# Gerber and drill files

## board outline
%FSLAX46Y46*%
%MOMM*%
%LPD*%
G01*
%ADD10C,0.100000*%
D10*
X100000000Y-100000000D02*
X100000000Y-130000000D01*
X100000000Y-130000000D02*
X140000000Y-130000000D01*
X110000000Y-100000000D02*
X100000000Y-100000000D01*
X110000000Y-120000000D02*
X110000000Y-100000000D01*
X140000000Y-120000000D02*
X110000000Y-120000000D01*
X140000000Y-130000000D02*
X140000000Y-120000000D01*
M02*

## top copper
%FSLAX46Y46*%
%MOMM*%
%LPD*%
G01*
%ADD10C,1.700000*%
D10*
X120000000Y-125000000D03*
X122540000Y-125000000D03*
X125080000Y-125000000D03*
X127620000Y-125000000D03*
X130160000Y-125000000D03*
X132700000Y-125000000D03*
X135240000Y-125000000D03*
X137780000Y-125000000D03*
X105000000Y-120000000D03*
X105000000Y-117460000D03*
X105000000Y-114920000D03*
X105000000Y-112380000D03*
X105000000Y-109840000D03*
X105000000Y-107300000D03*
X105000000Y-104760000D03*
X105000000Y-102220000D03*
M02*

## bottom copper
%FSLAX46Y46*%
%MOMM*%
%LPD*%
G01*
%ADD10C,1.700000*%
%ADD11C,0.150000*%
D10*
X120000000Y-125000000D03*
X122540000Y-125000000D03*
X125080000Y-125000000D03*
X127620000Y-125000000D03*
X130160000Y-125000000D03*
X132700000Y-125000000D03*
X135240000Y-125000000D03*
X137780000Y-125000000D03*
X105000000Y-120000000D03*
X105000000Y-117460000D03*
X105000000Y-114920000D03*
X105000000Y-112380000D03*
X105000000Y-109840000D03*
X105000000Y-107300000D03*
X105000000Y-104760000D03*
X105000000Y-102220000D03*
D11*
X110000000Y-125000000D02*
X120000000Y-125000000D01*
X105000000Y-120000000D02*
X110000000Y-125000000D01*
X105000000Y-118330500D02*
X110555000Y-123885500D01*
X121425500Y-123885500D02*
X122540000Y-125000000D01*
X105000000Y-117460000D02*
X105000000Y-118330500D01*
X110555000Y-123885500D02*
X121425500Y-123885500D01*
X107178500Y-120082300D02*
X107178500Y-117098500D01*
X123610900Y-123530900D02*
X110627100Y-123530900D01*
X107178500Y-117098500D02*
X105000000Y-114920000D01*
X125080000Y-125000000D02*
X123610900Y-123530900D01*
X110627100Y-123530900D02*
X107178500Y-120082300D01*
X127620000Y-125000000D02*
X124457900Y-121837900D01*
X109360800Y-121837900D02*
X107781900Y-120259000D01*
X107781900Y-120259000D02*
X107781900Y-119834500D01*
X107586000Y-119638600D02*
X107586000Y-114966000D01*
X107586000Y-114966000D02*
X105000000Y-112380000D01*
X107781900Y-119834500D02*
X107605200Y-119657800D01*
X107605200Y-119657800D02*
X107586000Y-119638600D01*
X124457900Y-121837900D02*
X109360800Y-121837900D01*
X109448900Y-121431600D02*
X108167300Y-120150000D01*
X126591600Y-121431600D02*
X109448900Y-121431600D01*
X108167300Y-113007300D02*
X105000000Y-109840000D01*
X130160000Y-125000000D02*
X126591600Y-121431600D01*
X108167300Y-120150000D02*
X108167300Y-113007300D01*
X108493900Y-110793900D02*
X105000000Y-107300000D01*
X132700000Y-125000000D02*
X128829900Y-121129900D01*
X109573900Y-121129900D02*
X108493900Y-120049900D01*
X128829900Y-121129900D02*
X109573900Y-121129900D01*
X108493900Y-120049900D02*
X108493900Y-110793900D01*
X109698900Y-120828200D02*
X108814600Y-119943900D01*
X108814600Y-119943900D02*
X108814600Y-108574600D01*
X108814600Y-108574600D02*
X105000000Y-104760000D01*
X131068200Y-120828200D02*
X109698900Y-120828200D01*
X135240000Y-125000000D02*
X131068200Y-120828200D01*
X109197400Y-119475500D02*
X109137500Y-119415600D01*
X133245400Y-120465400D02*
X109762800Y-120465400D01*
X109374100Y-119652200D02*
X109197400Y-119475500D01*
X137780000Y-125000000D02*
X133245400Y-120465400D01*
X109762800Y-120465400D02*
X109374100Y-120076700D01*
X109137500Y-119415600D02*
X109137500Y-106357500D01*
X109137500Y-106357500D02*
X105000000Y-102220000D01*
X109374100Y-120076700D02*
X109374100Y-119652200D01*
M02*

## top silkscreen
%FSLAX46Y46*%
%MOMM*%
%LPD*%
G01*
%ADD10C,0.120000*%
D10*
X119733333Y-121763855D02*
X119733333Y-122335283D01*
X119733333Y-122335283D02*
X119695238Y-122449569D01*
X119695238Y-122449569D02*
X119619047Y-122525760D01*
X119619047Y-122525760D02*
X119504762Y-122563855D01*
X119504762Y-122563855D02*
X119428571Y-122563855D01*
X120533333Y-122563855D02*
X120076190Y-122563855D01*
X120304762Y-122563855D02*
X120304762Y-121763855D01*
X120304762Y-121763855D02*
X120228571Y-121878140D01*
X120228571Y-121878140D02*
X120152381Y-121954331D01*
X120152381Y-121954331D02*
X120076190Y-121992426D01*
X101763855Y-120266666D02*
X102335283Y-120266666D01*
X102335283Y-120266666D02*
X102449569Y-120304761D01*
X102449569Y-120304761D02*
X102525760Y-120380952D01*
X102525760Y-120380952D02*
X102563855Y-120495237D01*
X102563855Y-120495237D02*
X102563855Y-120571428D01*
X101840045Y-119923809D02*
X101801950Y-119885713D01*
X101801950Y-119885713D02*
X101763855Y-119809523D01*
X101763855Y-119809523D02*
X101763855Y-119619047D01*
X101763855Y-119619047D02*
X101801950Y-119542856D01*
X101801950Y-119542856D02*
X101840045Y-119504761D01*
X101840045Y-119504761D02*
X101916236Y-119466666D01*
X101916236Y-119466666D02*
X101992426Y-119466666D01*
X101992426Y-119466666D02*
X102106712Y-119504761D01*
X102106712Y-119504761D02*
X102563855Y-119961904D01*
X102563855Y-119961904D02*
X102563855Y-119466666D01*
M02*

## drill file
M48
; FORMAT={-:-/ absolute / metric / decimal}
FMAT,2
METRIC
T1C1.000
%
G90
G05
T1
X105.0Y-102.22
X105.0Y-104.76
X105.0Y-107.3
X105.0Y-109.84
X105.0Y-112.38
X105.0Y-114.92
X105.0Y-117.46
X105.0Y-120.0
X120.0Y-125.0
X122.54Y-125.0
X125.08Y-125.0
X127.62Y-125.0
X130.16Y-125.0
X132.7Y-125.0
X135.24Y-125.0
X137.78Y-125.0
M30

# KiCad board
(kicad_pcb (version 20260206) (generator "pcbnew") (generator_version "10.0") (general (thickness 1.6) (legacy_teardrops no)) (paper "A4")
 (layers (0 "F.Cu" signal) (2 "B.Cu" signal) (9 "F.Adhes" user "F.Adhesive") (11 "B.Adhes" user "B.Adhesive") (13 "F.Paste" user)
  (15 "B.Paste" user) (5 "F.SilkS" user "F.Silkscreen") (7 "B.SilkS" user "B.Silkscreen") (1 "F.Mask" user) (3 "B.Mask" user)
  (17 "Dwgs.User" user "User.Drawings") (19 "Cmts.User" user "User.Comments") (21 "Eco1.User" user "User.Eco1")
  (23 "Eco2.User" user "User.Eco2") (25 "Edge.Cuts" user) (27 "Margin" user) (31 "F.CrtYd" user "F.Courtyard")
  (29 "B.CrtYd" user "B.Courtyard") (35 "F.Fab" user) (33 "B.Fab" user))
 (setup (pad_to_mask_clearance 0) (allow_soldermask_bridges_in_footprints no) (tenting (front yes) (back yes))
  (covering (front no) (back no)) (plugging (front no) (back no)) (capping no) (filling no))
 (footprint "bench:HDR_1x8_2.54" (layer "F.Cu") (at 120 125)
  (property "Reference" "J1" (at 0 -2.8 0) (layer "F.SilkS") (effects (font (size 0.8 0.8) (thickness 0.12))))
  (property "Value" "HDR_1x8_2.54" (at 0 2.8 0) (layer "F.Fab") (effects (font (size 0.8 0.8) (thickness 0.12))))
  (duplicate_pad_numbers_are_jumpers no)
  (pad "1" thru_hole circle (at 0 0) (size 1.7 1.7) (drill 1) (layers "*.Cu" "*.Mask") (remove_unused_layers no) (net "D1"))
  (pad "2" thru_hole circle (at 2.54 0) (size 1.7 1.7) (drill 1) (layers "*.Cu" "*.Mask") (remove_unused_layers no) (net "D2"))
  (pad "3" thru_hole circle (at 5.08 0) (size 1.7 1.7) (drill 1) (layers "*.Cu" "*.Mask") (remove_unused_layers no) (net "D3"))
  (pad "4" thru_hole circle (at 7.62 0) (size 1.7 1.7) (drill 1) (layers "*.Cu" "*.Mask") (remove_unused_layers no) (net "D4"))
  (pad "5" thru_hole circle (at 10.16 0) (size 1.7 1.7) (drill 1) (layers "*.Cu" "*.Mask") (remove_unused_layers no) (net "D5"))
  (pad "6" thru_hole circle (at 12.7 0) (size 1.7 1.7) (drill 1) (layers "*.Cu" "*.Mask") (remove_unused_layers no) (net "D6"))
  (pad "7" thru_hole circle (at 15.24 0) (size 1.7 1.7) (drill 1) (layers "*.Cu" "*.Mask") (remove_unused_layers no) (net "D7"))
  (pad "8" thru_hole circle (at 17.78 0) (size 1.7 1.7) (drill 1) (layers "*.Cu" "*.Mask") (remove_unused_layers no) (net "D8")))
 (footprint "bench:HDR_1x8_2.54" (layer "F.Cu") (at 105 120 90)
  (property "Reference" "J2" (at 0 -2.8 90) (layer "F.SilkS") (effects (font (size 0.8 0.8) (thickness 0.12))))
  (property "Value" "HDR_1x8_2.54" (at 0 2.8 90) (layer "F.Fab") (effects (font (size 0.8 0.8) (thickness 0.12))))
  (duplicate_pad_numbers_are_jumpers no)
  (pad "1" thru_hole circle (at 0 0 90) (size 1.7 1.7) (drill 1) (layers "*.Cu" "*.Mask") (remove_unused_layers no) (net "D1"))
  (pad "2" thru_hole circle (at 2.54 0 90) (size 1.7 1.7) (drill 1) (layers "*.Cu" "*.Mask") (remove_unused_layers no) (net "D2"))
  (pad "3" thru_hole circle (at 5.08 0 90) (size 1.7 1.7) (drill 1) (layers "*.Cu" "*.Mask") (remove_unused_layers no) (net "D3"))
  (pad "4" thru_hole circle (at 7.62 0 90) (size 1.7 1.7) (drill 1) (layers "*.Cu" "*.Mask") (remove_unused_layers no) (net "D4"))
  (pad "5" thru_hole circle (at 10.16 0 90) (size 1.7 1.7) (drill 1) (layers "*.Cu" "*.Mask") (remove_unused_layers no) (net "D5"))
  (pad "6" thru_hole circle (at 12.7 0 90) (size 1.7 1.7) (drill 1) (layers "*.Cu" "*.Mask") (remove_unused_layers no) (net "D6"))
  (pad "7" thru_hole circle (at 15.24 0 90) (size 1.7 1.7) (drill 1) (layers "*.Cu" "*.Mask") (remove_unused_layers no) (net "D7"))
  (pad "8" thru_hole circle (at 17.78 0 90) (size 1.7 1.7) (drill 1) (layers "*.Cu" "*.Mask") (remove_unused_layers no) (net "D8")))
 (gr_line (start 100 100) (end 100 130) (stroke (width 0.1) (type solid)) (layer "Edge.Cuts"))
 (gr_line (start 100 130) (end 140 130) (stroke (width 0.1) (type solid)) (layer "Edge.Cuts"))
 (gr_line (start 110 100) (end 100 100) (stroke (width 0.1) (type solid)) (layer "Edge.Cuts"))
 (gr_line (start 110 120) (end 110 100) (stroke (width 0.1) (type solid)) (layer "Edge.Cuts"))
 (gr_line (start 140 120) (end 110 120) (stroke (width 0.1) (type solid)) (layer "Edge.Cuts"))
 (gr_line (start 140 130) (end 140 120) (stroke (width 0.1) (type solid)) (layer "Edge.Cuts"))
 (segment (start 110 125) (end 120 125) (width 0.15) (layer "B.Cu") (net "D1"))
 (segment (start 105 120) (end 110 125) (width 0.15) (layer "B.Cu") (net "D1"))
 (segment (start 105 118.3305) (end 110.555 123.8855) (width 0.15) (layer "B.Cu") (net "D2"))
 (segment (start 121.4255 123.8855) (end 122.54 125) (width 0.15) (layer "B.Cu") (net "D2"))
 (segment (start 105 117.46) (end 105 118.3305) (width 0.15) (layer "B.Cu") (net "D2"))
 (segment (start 110.555 123.8855) (end 121.4255 123.8855) (width 0.15) (layer "B.Cu") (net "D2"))
 (segment (start 107.1785 120.0823) (end 107.1785 117.0985) (width 0.15) (layer "B.Cu") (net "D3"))
 (segment (start 123.6109 123.5309) (end 110.6271 123.5309) (width 0.15) (layer "B.Cu") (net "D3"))
 (segment (start 107.1785 117.0985) (end 105 114.92) (width 0.15) (layer "B.Cu") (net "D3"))
 (segment (start 125.08 125) (end 123.6109 123.5309) (width 0.15) (layer "B.Cu") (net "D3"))
 (segment (start 110.6271 123.5309) (end 107.1785 120.0823) (width 0.15) (layer "B.Cu") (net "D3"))
 (segment (start 127.62 125) (end 124.4579 121.8379) (width 0.15) (layer "B.Cu") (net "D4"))
 (segment (start 109.3608 121.8379) (end 107.7819 120.259) (width 0.15) (layer "B.Cu") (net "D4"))
 (segment (start 107.7819 120.259) (end 107.7819 119.8345) (width 0.15) (layer "B.Cu") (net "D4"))
 (segment (start 107.586 119.6386) (end 107.586 114.966) (width 0.15) (layer "B.Cu") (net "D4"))
 (segment (start 107.586 114.966) (end 105 112.38) (width 0.15) (layer "B.Cu") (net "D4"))
 (segment (start 107.7819 119.8345) (end 107.6052 119.6578) (width 0.15) (layer "B.Cu") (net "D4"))
 (segment (start 107.6052 119.6578) (end 107.586 119.6386) (width 0.15) (layer "B.Cu") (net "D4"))
 (segment (start 124.4579 121.8379) (end 109.3608 121.8379) (width 0.15) (layer "B.Cu") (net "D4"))
 (segment (start 109.4489 121.4316) (end 108.1673 120.15) (width 0.15) (layer "B.Cu") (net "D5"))
 (segment (start 126.5916 121.4316) (end 109.4489 121.4316) (width 0.15) (layer "B.Cu") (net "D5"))
 (segment (start 108.1673 113.0073) (end 105 109.84) (width 0.15) (layer "B.Cu") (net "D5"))
 (segment (start 130.16 125) (end 126.5916 121.4316) (width 0.15) (layer "B.Cu") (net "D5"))
 (segment (start 108.1673 120.15) (end 108.1673 113.0073) (width 0.15) (layer "B.Cu") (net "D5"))
 (segment (start 108.4939 110.7939) (end 105 107.3) (width 0.15) (layer "B.Cu") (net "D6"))
 (segment (start 132.7 125) (end 128.8299 121.1299) (width 0.15) (layer "B.Cu") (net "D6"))
 (segment (start 109.5739 121.1299) (end 108.4939 120.0499) (width 0.15) (layer "B.Cu") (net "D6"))
 (segment (start 128.8299 121.1299) (end 109.5739 121.1299) (width 0.15) (layer "B.Cu") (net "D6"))
 (segment (start 108.4939 120.0499) (end 108.4939 110.7939) (width 0.15) (layer "B.Cu") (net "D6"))
 (segment (start 109.6989 120.8282) (end 108.8146 119.9439) (width 0.15) (layer "B.Cu") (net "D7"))
 (segment (start 108.8146 119.9439) (end 108.8146 108.5746) (width 0.15) (layer "B.Cu") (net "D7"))
 (segment (start 108.8146 108.5746) (end 105 104.76) (width 0.15) (layer "B.Cu") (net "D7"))
 (segment (start 131.0682 120.8282) (end 109.6989 120.8282) (width 0.15) (layer "B.Cu") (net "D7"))
 (segment (start 135.24 125) (end 131.0682 120.8282) (width 0.15) (layer "B.Cu") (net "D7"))
 (segment (start 109.1974 119.4755) (end 109.1375 119.4156) (width 0.15) (layer "B.Cu") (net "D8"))
 (segment (start 133.2454 120.4654) (end 109.7628 120.4654) (width 0.15) (layer "B.Cu") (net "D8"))
 (segment (start 109.3741 119.6522) (end 109.1974 119.4755) (width 0.15) (layer "B.Cu") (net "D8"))
 (segment (start 137.78 125) (end 133.2454 120.4654) (width 0.15) (layer "B.Cu") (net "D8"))
 (segment (start 109.7628 120.4654) (end 109.3741 120.0767) (width 0.15) (layer "B.Cu") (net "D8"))
 (segment (start 109.1375 119.4156) (end 109.1375 106.3575) (width 0.15) (layer "B.Cu") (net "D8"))
 (segment (start 109.1375 106.3575) (end 105 102.22) (width 0.15) (layer "B.Cu") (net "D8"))
 (segment (start 109.3741 120.0767) (end 109.3741 119.6522) (width 0.15) (layer "B.Cu") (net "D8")))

